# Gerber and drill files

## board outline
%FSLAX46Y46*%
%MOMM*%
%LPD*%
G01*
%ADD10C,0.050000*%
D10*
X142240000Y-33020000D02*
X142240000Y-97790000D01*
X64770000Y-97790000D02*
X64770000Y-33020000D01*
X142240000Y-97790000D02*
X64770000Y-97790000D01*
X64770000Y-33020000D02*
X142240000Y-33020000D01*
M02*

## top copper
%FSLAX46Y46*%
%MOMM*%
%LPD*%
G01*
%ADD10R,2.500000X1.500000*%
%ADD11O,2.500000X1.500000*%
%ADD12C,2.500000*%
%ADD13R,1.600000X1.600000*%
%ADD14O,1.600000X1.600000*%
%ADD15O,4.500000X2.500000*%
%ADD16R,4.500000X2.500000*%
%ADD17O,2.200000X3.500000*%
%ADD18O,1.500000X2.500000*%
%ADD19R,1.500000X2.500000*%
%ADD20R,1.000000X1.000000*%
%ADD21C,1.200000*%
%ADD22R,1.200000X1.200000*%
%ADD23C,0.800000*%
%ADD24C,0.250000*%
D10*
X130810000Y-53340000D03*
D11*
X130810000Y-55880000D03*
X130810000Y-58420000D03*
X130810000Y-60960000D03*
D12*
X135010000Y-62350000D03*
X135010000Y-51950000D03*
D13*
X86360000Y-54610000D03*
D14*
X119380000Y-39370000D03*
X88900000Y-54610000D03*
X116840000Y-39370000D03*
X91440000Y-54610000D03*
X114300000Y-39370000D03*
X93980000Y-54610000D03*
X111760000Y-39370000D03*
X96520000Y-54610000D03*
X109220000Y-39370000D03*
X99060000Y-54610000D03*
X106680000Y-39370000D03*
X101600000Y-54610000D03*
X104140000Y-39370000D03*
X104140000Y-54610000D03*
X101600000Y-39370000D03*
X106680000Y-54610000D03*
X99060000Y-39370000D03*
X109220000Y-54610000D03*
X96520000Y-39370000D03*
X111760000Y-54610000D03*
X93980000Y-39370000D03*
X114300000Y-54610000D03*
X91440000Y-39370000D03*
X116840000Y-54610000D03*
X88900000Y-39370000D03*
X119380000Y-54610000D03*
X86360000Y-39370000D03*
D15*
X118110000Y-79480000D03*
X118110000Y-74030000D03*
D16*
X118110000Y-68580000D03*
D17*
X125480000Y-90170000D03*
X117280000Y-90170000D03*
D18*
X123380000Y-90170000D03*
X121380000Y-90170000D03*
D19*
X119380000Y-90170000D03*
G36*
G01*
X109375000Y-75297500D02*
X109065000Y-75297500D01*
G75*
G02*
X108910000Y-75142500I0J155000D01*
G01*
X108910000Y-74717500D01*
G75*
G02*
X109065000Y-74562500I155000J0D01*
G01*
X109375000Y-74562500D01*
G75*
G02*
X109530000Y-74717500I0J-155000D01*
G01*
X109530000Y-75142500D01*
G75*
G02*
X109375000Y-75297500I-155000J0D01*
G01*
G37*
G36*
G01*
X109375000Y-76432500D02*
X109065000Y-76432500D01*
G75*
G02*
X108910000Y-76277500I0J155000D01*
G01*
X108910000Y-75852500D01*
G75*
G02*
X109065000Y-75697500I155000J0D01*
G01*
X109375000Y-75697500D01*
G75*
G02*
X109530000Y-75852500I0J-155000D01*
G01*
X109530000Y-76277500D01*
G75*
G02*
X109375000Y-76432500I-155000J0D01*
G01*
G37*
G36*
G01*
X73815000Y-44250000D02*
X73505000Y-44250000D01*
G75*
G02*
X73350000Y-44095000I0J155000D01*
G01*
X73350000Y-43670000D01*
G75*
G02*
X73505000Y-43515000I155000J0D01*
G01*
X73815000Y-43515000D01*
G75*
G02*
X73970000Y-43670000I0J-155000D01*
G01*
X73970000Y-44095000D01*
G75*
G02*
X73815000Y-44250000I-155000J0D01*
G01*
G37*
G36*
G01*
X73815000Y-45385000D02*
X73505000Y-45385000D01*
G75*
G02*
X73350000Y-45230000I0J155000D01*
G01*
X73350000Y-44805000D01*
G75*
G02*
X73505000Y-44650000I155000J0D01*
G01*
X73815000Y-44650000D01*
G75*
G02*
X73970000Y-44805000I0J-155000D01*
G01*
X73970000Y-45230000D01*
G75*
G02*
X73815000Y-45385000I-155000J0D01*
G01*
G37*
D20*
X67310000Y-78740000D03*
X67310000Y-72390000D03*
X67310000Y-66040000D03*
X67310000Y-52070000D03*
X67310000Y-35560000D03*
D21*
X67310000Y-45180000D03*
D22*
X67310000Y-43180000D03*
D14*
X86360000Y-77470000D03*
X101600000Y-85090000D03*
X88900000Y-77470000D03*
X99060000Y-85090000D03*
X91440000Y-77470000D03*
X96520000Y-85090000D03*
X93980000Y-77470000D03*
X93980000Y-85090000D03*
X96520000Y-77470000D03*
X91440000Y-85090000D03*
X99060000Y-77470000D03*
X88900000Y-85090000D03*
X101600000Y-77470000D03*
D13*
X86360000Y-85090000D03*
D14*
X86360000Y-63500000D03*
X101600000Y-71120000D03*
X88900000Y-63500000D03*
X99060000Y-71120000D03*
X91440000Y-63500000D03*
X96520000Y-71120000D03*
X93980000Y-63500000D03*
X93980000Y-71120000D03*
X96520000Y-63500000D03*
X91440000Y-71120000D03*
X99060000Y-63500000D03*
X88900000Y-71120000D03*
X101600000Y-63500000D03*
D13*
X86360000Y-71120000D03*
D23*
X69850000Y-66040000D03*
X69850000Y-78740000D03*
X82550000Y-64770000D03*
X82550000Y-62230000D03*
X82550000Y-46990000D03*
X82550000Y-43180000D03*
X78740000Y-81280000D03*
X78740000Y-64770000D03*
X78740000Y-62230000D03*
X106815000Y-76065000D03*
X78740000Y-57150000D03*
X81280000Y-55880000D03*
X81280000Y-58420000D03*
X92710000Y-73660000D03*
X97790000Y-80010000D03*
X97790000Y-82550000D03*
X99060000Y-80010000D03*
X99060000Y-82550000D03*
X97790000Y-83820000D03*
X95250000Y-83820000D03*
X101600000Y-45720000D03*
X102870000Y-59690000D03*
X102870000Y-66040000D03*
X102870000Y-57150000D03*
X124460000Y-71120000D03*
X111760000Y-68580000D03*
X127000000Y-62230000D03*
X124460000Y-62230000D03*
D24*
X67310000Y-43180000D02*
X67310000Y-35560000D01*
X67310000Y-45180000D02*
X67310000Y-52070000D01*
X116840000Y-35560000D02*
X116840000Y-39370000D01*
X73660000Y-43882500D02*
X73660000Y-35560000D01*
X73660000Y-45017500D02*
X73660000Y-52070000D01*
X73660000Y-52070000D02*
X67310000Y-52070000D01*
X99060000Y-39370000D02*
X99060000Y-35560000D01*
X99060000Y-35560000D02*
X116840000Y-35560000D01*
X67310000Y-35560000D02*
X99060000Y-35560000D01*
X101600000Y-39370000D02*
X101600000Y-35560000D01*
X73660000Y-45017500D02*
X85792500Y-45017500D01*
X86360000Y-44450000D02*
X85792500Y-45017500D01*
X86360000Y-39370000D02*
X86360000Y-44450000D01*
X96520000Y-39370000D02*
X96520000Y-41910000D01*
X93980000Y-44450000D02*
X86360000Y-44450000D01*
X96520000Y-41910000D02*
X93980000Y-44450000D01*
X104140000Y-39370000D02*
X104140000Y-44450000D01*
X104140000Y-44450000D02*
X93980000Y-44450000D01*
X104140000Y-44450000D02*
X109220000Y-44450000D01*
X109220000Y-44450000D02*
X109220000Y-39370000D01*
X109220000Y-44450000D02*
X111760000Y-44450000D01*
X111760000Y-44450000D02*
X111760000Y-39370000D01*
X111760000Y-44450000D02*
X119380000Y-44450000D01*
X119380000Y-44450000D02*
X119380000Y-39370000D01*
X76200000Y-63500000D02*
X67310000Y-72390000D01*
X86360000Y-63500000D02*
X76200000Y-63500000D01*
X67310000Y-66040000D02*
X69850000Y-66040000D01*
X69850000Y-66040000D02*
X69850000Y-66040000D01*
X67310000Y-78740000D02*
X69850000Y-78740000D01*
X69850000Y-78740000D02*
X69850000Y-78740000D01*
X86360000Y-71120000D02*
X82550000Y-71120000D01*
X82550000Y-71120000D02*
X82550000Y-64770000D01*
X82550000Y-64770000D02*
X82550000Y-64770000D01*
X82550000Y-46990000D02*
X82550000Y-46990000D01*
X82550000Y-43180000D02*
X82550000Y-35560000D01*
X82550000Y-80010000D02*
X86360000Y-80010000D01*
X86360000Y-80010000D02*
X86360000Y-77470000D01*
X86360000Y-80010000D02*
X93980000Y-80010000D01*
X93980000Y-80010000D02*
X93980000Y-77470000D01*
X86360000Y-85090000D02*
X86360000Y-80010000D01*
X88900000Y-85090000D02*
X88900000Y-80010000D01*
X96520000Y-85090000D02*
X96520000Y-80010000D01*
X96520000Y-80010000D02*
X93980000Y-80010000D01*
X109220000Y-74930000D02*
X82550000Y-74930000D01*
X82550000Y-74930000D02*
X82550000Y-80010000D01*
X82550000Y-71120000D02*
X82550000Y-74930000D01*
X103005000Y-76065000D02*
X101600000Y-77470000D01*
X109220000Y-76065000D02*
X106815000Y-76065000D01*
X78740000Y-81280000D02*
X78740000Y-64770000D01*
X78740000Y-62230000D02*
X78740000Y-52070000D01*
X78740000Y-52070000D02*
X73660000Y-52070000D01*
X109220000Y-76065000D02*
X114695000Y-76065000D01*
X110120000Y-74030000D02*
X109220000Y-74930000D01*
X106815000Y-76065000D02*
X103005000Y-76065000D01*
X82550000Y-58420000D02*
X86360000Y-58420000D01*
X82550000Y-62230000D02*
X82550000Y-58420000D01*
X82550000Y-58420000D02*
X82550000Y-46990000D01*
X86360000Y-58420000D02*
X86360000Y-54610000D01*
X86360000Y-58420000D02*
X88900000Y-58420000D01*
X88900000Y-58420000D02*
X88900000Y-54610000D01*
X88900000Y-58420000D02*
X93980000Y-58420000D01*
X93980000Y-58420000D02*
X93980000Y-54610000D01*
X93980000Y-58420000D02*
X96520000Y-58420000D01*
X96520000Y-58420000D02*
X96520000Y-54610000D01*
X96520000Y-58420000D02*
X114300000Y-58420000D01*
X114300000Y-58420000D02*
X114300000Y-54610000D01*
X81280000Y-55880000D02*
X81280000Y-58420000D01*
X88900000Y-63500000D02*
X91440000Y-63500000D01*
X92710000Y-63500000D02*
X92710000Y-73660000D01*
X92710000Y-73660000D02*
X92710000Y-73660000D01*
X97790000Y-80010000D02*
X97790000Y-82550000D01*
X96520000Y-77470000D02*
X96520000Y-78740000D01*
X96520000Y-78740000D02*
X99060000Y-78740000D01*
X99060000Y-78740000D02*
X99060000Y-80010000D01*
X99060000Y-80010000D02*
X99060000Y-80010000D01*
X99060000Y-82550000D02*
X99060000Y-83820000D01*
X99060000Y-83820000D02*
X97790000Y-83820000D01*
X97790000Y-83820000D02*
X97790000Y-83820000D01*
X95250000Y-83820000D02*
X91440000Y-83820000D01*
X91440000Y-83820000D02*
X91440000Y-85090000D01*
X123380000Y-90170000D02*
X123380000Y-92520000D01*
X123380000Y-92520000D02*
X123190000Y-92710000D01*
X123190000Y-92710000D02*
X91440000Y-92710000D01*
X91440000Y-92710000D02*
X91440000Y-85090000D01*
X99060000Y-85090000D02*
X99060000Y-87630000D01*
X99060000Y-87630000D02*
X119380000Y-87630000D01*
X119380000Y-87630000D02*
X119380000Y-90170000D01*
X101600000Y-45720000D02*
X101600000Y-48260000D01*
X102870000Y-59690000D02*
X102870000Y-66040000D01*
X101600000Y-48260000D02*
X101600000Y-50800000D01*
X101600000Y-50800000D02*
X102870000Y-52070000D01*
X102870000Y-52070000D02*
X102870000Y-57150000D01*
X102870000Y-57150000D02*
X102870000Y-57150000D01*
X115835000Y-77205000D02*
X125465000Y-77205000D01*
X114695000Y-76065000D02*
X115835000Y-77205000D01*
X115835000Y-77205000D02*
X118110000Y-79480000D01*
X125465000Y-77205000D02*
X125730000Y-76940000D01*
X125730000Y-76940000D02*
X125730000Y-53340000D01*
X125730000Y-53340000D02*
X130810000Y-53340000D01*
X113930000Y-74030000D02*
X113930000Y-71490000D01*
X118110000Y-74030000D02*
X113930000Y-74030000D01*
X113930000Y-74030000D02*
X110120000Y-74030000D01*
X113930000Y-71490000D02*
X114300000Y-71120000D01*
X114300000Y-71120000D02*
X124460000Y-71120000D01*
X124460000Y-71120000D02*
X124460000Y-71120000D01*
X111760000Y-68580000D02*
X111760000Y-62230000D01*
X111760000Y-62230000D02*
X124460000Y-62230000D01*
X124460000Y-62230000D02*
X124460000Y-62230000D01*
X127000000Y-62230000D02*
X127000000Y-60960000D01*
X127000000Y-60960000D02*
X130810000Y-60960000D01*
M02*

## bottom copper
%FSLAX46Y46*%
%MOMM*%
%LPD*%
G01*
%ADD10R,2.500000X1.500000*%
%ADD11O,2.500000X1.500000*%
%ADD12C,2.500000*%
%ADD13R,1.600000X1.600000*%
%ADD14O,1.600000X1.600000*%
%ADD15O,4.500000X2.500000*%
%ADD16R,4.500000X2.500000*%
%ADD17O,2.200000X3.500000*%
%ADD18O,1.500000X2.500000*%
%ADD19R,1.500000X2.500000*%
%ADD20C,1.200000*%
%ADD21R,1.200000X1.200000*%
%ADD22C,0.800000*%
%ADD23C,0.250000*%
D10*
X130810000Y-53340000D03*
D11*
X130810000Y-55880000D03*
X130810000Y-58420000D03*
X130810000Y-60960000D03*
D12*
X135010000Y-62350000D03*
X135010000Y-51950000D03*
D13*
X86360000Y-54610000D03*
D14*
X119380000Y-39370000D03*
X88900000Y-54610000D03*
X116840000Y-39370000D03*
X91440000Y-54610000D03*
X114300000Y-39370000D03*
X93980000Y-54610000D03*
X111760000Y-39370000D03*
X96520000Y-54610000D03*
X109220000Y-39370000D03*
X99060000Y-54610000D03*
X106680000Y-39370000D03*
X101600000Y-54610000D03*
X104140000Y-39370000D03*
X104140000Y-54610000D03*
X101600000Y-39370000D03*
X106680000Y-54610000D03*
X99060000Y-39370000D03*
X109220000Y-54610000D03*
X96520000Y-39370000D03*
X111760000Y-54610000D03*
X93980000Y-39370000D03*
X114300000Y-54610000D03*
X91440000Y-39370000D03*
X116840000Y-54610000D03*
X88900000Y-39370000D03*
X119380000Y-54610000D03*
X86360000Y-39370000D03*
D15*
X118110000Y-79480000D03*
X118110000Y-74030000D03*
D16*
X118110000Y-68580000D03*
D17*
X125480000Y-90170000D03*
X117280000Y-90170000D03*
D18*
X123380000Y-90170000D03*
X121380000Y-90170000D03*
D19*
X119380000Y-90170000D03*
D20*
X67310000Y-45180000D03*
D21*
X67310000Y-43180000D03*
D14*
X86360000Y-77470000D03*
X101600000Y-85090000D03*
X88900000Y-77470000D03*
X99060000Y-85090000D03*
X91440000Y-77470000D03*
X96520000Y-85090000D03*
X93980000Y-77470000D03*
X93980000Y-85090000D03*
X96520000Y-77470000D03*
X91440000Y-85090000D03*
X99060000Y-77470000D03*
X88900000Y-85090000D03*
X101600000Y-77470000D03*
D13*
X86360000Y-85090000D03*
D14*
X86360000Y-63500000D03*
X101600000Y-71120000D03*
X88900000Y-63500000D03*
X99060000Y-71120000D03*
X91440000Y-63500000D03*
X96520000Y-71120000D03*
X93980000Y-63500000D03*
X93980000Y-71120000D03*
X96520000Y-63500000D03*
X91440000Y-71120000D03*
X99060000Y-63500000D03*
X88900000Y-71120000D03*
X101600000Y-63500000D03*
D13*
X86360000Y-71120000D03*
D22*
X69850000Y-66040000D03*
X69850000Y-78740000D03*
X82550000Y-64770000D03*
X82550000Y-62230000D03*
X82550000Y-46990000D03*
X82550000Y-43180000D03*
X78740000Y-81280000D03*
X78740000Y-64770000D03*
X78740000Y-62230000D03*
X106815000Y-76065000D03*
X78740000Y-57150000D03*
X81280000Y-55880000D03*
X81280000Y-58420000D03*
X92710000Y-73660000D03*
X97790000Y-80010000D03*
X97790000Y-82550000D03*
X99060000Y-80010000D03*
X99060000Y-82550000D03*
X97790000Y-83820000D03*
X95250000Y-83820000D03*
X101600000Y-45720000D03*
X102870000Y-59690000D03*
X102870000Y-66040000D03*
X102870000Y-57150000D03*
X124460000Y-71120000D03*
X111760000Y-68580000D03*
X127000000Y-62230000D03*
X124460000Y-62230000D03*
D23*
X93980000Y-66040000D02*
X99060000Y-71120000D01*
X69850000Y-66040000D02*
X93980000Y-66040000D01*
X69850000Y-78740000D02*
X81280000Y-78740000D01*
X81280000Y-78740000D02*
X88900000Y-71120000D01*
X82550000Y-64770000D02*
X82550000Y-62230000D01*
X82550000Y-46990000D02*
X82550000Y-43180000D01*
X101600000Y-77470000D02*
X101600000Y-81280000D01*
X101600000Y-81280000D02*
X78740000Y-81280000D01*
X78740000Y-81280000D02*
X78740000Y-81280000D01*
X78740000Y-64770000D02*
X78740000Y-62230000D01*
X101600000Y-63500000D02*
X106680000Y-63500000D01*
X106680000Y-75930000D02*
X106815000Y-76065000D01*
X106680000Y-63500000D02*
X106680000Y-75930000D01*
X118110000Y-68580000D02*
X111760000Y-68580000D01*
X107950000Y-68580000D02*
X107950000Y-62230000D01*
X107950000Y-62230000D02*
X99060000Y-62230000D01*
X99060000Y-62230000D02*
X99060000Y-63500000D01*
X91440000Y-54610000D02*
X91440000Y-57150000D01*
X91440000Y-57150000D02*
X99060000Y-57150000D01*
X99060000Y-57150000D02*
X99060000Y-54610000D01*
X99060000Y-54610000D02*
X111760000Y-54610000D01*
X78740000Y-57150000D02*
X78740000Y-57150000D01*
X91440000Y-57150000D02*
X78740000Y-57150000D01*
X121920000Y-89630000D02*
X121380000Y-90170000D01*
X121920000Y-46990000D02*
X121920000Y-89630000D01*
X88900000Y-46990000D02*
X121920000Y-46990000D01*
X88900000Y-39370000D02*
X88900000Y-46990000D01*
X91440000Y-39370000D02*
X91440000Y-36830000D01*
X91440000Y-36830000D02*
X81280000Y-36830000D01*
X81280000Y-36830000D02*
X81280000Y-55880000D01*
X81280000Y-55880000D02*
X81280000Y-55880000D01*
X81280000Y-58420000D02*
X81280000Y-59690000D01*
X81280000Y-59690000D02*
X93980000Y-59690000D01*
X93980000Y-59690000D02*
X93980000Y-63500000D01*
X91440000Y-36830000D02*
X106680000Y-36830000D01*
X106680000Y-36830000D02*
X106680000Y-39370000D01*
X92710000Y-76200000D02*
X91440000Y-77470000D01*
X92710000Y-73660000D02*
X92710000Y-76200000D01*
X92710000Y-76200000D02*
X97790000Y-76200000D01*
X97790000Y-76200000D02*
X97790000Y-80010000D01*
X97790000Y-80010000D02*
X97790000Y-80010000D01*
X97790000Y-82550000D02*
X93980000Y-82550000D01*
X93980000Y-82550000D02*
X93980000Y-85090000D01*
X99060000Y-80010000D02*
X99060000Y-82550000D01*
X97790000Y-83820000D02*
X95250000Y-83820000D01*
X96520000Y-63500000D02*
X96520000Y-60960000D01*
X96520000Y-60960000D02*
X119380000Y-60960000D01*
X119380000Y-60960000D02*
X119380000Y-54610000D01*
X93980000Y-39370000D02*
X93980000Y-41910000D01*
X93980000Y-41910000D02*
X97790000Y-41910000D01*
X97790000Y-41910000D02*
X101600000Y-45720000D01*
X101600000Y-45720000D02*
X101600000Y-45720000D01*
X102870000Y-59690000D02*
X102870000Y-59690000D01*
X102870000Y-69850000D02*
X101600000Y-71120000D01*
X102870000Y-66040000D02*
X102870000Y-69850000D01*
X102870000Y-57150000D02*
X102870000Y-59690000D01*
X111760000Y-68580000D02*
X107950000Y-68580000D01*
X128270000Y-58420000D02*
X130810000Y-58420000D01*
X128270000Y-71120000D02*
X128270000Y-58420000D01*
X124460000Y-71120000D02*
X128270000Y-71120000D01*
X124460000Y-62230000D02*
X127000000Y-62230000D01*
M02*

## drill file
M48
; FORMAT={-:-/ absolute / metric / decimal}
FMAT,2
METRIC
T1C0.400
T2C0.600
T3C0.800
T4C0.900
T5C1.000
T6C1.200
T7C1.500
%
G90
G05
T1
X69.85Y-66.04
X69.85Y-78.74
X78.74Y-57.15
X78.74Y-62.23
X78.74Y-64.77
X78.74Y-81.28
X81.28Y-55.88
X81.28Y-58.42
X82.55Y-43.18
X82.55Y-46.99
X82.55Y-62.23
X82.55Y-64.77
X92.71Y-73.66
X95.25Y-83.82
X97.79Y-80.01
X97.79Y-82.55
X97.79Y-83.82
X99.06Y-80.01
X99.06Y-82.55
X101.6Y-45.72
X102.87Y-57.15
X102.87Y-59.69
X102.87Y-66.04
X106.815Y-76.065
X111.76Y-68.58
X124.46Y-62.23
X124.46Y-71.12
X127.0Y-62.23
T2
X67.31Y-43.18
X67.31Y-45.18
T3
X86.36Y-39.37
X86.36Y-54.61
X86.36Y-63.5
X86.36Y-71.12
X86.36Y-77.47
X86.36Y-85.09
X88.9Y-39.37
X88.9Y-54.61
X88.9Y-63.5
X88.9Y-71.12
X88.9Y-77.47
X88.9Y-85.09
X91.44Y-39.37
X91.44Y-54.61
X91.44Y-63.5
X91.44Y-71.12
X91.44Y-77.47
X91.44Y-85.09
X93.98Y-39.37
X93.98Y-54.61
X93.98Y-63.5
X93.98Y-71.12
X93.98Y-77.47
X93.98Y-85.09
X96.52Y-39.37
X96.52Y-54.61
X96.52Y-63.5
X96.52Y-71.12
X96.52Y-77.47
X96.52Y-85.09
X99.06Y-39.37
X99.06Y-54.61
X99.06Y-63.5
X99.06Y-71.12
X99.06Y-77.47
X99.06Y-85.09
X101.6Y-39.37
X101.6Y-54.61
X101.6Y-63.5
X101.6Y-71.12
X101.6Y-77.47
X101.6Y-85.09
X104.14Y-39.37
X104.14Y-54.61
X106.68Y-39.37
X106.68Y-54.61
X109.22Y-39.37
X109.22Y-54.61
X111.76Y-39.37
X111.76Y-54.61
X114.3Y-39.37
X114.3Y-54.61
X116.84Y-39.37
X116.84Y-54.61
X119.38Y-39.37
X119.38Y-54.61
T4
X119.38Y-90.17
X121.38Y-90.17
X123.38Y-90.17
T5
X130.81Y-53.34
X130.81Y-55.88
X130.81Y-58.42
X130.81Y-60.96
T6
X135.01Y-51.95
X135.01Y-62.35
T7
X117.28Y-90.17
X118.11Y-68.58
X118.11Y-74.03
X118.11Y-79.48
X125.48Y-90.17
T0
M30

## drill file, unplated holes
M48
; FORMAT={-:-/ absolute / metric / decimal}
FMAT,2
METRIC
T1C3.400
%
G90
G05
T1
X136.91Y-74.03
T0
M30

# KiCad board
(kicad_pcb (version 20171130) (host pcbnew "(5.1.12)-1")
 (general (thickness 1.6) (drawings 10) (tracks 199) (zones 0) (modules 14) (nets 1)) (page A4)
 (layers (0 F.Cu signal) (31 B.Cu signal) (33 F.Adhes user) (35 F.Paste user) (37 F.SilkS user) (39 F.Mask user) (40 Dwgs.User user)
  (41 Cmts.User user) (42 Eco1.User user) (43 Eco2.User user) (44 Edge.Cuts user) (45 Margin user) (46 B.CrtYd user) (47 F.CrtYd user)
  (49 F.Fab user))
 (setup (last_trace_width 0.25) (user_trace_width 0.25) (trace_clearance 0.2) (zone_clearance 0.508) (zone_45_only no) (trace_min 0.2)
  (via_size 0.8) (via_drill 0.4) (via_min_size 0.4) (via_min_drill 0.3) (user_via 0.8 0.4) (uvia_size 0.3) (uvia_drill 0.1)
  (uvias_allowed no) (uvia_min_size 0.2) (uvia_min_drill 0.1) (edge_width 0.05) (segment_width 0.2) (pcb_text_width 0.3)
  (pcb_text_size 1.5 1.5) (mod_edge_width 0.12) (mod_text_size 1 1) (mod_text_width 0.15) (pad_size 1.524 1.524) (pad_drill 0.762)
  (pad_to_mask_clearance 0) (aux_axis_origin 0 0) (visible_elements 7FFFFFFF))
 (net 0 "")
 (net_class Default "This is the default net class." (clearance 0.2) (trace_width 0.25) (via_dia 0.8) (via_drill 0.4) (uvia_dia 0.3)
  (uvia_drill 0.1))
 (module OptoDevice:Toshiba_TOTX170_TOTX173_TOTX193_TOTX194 (layer F.Cu) (at 130.81 53.34 270)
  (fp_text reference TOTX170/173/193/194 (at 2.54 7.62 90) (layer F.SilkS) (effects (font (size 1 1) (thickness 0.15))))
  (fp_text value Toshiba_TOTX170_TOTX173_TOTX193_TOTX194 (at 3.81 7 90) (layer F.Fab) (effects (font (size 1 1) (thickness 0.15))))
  (pad 1 thru_hole rect (at 0 0 270) (size 1.5 2.5) (drill 1) (layers *.Cu *.Mask))
  (pad 2 thru_hole oval (at 2.54 0 270) (size 1.5 2.5) (drill 1) (layers *.Cu *.Mask))
  (pad 3 thru_hole oval (at 5.08 0 270) (size 1.5 2.5) (drill 1) (layers *.Cu *.Mask))
  (pad 4 thru_hole oval (at 7.62 0 270) (size 1.5 2.5) (drill 1) (layers *.Cu *.Mask))
  (pad 5 thru_hole circle (at 9.01 -4.2 270) (size 2.5 2.5) (drill 1.2) (layers *.Cu *.Mask))
  (pad 6 thru_hole circle (at -1.39 -4.2 270) (size 2.5 2.5) (drill 1.2) (layers *.Cu *.Mask)))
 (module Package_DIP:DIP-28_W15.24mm (layer F.Cu) (at 86.36 54.61 90)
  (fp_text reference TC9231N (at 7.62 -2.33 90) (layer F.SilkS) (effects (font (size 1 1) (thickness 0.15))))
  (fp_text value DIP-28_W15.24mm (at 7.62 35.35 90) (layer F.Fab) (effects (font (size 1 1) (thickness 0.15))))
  (pad 1 thru_hole rect (at 0 0 90) (size 1.6 1.6) (drill 0.8) (layers *.Cu *.Mask))
  (pad 15 thru_hole oval (at 15.24 33.02 90) (size 1.6 1.6) (drill 0.8) (layers *.Cu *.Mask))
  (pad 2 thru_hole oval (at 0 2.54 90) (size 1.6 1.6) (drill 0.8) (layers *.Cu *.Mask))
  (pad 16 thru_hole oval (at 15.24 30.48 90) (size 1.6 1.6) (drill 0.8) (layers *.Cu *.Mask))
  (pad 3 thru_hole oval (at 0 5.08 90) (size 1.6 1.6) (drill 0.8) (layers *.Cu *.Mask))
  (pad 17 thru_hole oval (at 15.24 27.94 90) (size 1.6 1.6) (drill 0.8) (layers *.Cu *.Mask))
  (pad 4 thru_hole oval (at 0 7.62 90) (size 1.6 1.6) (drill 0.8) (layers *.Cu *.Mask))
  (pad 18 thru_hole oval (at 15.24 25.4 90) (size 1.6 1.6) (drill 0.8) (layers *.Cu *.Mask))
  (pad 5 thru_hole oval (at 0 10.16 90) (size 1.6 1.6) (drill 0.8) (layers *.Cu *.Mask))
  (pad 19 thru_hole oval (at 15.24 22.86 90) (size 1.6 1.6) (drill 0.8) (layers *.Cu *.Mask))
  (pad 6 thru_hole oval (at 0 12.7 90) (size 1.6 1.6) (drill 0.8) (layers *.Cu *.Mask))
  (pad 20 thru_hole oval (at 15.24 20.32 90) (size 1.6 1.6) (drill 0.8) (layers *.Cu *.Mask))
  (pad 7 thru_hole oval (at 0 15.24 90) (size 1.6 1.6) (drill 0.8) (layers *.Cu *.Mask))
  (pad 21 thru_hole oval (at 15.24 17.78 90) (size 1.6 1.6) (drill 0.8) (layers *.Cu *.Mask))
  (pad 8 thru_hole oval (at 0 17.78 90) (size 1.6 1.6) (drill 0.8) (layers *.Cu *.Mask))
  (pad 22 thru_hole oval (at 15.24 15.24 90) (size 1.6 1.6) (drill 0.8) (layers *.Cu *.Mask))
  (pad 9 thru_hole oval (at 0 20.32 90) (size 1.6 1.6) (drill 0.8) (layers *.Cu *.Mask))
  (pad 23 thru_hole oval (at 15.24 12.7 90) (size 1.6 1.6) (drill 0.8) (layers *.Cu *.Mask))
  (pad 10 thru_hole oval (at 0 22.86 90) (size 1.6 1.6) (drill 0.8) (layers *.Cu *.Mask))
  (pad 24 thru_hole oval (at 15.24 10.16 90) (size 1.6 1.6) (drill 0.8) (layers *.Cu *.Mask))
  (pad 11 thru_hole oval (at 0 25.4 90) (size 1.6 1.6) (drill 0.8) (layers *.Cu *.Mask))
  (pad 25 thru_hole oval (at 15.24 7.62 90) (size 1.6 1.6) (drill 0.8) (layers *.Cu *.Mask))
  (pad 12 thru_hole oval (at 0 27.94 90) (size 1.6 1.6) (drill 0.8) (layers *.Cu *.Mask))
  (pad 26 thru_hole oval (at 15.24 5.08 90) (size 1.6 1.6) (drill 0.8) (layers *.Cu *.Mask))
  (pad 13 thru_hole oval (at 0 30.48 90) (size 1.6 1.6) (drill 0.8) (layers *.Cu *.Mask))
  (pad 27 thru_hole oval (at 15.24 2.54 90) (size 1.6 1.6) (drill 0.8) (layers *.Cu *.Mask))
  (pad 14 thru_hole oval (at 0 33.02 90) (size 1.6 1.6) (drill 0.8) (layers *.Cu *.Mask))
  (pad 28 thru_hole oval (at 15.24 0 90) (size 1.6 1.6) (drill 0.8) (layers *.Cu *.Mask)))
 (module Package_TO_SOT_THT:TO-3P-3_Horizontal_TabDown (layer F.Cu) (at 118.11 68.58 270)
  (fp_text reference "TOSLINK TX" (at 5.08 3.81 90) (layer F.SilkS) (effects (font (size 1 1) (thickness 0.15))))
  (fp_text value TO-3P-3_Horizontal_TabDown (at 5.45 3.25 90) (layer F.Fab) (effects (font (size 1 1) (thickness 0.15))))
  (pad 3 thru_hole oval (at 10.9 0 270) (size 2.5 4.5) (drill 1.5) (layers *.Cu *.Mask))
  (pad 2 thru_hole oval (at 5.45 0 270) (size 2.5 4.5) (drill 1.5) (layers *.Cu *.Mask))
  (pad 1 thru_hole rect (at 0 0 270) (size 2.5 4.5) (drill 1.5) (layers *.Cu *.Mask))
  (pad "" np_thru_hole oval (at 5.45 -18.8 270) (size 3.4 3.4) (drill 3.4) (layers *.Cu *.Mask)))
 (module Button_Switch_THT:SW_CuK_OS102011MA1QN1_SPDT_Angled (layer F.Cu) (at 119.38 90.17)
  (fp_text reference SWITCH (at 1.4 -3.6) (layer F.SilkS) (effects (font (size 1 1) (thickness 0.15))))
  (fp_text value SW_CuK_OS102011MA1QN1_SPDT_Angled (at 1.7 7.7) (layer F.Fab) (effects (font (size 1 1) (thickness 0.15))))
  (pad "" thru_hole oval (at 6.1 0) (size 2.2 3.5) (drill 1.5) (layers *.Cu *.Mask))
  (pad "" thru_hole oval (at -2.1 0) (size 2.2 3.5) (drill 1.5) (layers *.Cu *.Mask))
  (pad 3 thru_hole oval (at 4 0) (size 1.5 2.5) (drill 0.9) (layers *.Cu *.Mask))
  (pad 2 thru_hole oval (at 2 0) (size 1.5 2.5) (drill 0.9) (layers *.Cu *.Mask))
  (pad 1 thru_hole rect (at 0 0) (size 1.5 2.5) (drill 0.9) (layers *.Cu *.Mask)))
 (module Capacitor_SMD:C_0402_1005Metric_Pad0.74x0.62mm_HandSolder (layer F.Cu) (at 109.22 75.4975 90)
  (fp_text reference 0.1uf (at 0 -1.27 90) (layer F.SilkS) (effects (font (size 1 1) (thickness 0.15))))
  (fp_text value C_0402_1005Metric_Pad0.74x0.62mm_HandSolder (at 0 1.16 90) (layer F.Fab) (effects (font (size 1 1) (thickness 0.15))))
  (pad 2 smd roundrect (at 0.5675 0 90) (size 0.735 0.62) (layers F.Cu F.Paste F.Mask) (roundrect_rratio 0.25))
  (pad 1 smd roundrect (at -0.5675 0 90) (size 0.735 0.62) (layers F.Cu F.Paste F.Mask) (roundrect_rratio 0.25)))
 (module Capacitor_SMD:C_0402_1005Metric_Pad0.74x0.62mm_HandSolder (layer F.Cu) (at 73.66 44.45 90)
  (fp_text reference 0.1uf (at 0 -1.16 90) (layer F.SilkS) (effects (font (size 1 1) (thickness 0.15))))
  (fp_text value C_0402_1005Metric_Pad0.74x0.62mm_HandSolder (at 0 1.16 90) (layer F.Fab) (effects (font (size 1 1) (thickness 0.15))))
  (pad 2 smd roundrect (at 0.5675 0 90) (size 0.735 0.62) (layers F.Cu F.Paste F.Mask) (roundrect_rratio 0.25))
  (pad 1 smd roundrect (at -0.5675 0 90) (size 0.735 0.62) (layers F.Cu F.Paste F.Mask) (roundrect_rratio 0.25)))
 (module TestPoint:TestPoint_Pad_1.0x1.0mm (layer F.Cu) (at 67.31 78.74)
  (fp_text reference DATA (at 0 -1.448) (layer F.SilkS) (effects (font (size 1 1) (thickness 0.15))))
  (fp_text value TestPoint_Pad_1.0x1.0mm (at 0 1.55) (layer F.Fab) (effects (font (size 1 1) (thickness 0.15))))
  (pad 1 smd rect (at 0 0) (size 1 1) (layers F.Cu F.Mask)))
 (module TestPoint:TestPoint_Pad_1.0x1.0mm (layer F.Cu) (at 67.31 72.39)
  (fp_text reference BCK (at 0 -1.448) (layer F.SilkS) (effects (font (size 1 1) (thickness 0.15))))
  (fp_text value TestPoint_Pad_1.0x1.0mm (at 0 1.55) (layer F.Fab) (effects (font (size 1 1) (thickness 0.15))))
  (pad 1 smd rect (at 0 0) (size 1 1) (layers F.Cu F.Mask)))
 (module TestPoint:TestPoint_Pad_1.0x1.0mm (layer F.Cu) (at 67.31 66.04)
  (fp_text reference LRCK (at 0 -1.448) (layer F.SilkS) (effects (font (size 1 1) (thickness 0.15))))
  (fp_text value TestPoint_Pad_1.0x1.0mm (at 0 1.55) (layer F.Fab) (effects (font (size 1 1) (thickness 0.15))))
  (pad 1 smd rect (at 0 0) (size 1 1) (layers F.Cu F.Mask)))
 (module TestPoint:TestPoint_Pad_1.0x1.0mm (layer F.Cu) (at 67.31 52.07)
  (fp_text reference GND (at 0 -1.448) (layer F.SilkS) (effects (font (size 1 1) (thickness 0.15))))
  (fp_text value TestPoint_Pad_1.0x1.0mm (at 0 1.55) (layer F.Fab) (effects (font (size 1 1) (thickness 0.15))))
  (pad 1 smd rect (at 0 0) (size 1 1) (layers F.Cu F.Mask)))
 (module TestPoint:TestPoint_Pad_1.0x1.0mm (layer F.Cu) (at 67.31 35.56)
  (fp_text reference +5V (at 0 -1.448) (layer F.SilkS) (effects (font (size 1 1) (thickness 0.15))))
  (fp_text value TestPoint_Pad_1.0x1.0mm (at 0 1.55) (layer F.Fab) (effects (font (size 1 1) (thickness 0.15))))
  (pad 1 smd rect (at 0 0) (size 1 1) (layers F.Cu F.Mask)))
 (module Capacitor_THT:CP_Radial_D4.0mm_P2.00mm (layer F.Cu) (at 67.31 43.18 270)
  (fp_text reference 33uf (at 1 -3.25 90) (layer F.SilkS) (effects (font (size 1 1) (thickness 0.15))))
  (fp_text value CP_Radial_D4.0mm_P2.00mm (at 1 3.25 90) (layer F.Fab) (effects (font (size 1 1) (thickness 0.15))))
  (pad 2 thru_hole circle (at 2 0 270) (size 1.2 1.2) (drill 0.6) (layers *.Cu *.Mask))
  (pad 1 thru_hole rect (at 0 0 270) (size 1.2 1.2) (drill 0.6) (layers *.Cu *.Mask)))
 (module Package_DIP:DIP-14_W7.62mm (layer F.Cu) (at 86.36 85.09 90)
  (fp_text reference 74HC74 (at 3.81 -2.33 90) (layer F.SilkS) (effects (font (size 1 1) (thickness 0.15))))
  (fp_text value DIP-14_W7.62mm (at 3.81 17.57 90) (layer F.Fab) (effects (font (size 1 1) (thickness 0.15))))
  (pad 14 thru_hole oval (at 7.62 0 90) (size 1.6 1.6) (drill 0.8) (layers *.Cu *.Mask))
  (pad 7 thru_hole oval (at 0 15.24 90) (size 1.6 1.6) (drill 0.8) (layers *.Cu *.Mask))
  (pad 13 thru_hole oval (at 7.62 2.54 90) (size 1.6 1.6) (drill 0.8) (layers *.Cu *.Mask))
  (pad 6 thru_hole oval (at 0 12.7 90) (size 1.6 1.6) (drill 0.8) (layers *.Cu *.Mask))
  (pad 12 thru_hole oval (at 7.62 5.08 90) (size 1.6 1.6) (drill 0.8) (layers *.Cu *.Mask))
  (pad 5 thru_hole oval (at 0 10.16 90) (size 1.6 1.6) (drill 0.8) (layers *.Cu *.Mask))
  (pad 11 thru_hole oval (at 7.62 7.62 90) (size 1.6 1.6) (drill 0.8) (layers *.Cu *.Mask))
  (pad 4 thru_hole oval (at 0 7.62 90) (size 1.6 1.6) (drill 0.8) (layers *.Cu *.Mask))
  (pad 10 thru_hole oval (at 7.62 10.16 90) (size 1.6 1.6) (drill 0.8) (layers *.Cu *.Mask))
  (pad 3 thru_hole oval (at 0 5.08 90) (size 1.6 1.6) (drill 0.8) (layers *.Cu *.Mask))
  (pad 9 thru_hole oval (at 7.62 12.7 90) (size 1.6 1.6) (drill 0.8) (layers *.Cu *.Mask))
  (pad 2 thru_hole oval (at 0 2.54 90) (size 1.6 1.6) (drill 0.8) (layers *.Cu *.Mask))
  (pad 8 thru_hole oval (at 7.62 15.24 90) (size 1.6 1.6) (drill 0.8) (layers *.Cu *.Mask))
  (pad 1 thru_hole rect (at 0 0 90) (size 1.6 1.6) (drill 0.8) (layers *.Cu *.Mask)))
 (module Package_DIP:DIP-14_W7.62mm (layer F.Cu) (at 86.36 71.12 90)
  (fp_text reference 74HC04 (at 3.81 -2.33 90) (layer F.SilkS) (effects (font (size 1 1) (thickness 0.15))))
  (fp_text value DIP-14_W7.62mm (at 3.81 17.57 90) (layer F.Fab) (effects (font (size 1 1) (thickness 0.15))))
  (pad 14 thru_hole oval (at 7.62 0 90) (size 1.6 1.6) (drill 0.8) (layers *.Cu *.Mask))
  (pad 7 thru_hole oval (at 0 15.24 90) (size 1.6 1.6) (drill 0.8) (layers *.Cu *.Mask))
  (pad 13 thru_hole oval (at 7.62 2.54 90) (size 1.6 1.6) (drill 0.8) (layers *.Cu *.Mask))
  (pad 6 thru_hole oval (at 0 12.7 90) (size 1.6 1.6) (drill 0.8) (layers *.Cu *.Mask))
  (pad 12 thru_hole oval (at 7.62 5.08 90) (size 1.6 1.6) (drill 0.8) (layers *.Cu *.Mask))
  (pad 5 thru_hole oval (at 0 10.16 90) (size 1.6 1.6) (drill 0.8) (layers *.Cu *.Mask))
  (pad 11 thru_hole oval (at 7.62 7.62 90) (size 1.6 1.6) (drill 0.8) (layers *.Cu *.Mask))
  (pad 4 thru_hole oval (at 0 7.62 90) (size 1.6 1.6) (drill 0.8) (layers *.Cu *.Mask))
  (pad 10 thru_hole oval (at 7.62 10.16 90) (size 1.6 1.6) (drill 0.8) (layers *.Cu *.Mask))
  (pad 3 thru_hole oval (at 0 5.08 90) (size 1.6 1.6) (drill 0.8) (layers *.Cu *.Mask))
  (pad 9 thru_hole oval (at 7.62 12.7 90) (size 1.6 1.6) (drill 0.8) (layers *.Cu *.Mask))
  (pad 2 thru_hole oval (at 0 2.54 90) (size 1.6 1.6) (drill 0.8) (layers *.Cu *.Mask))
  (pad 8 thru_hole oval (at 7.62 15.24 90) (size 1.6 1.6) (drill 0.8) (layers *.Cu *.Mask))
  (pad 1 thru_hole rect (at 0 0 90) (size 1.6 1.6) (drill 0.8) (layers *.Cu *.Mask)))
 (gr_line (start 142.24 33.02) (end 142.24 97.79) (layer Edge.Cuts) (width 0.05))
 (gr_line (start 64.77 97.79) (end 64.77 33.02) (layer Edge.Cuts) (width 0.05))
 (gr_line (start 142.24 97.79) (end 64.77 97.79) (layer Edge.Cuts) (width 0.05))
 (gr_line (start 64.77 33.02) (end 142.24 33.02) (layer Edge.Cuts) (width 0.05))
 (segment (start 67.31 43.18) (end 67.31 35.56) (width 0.25) (layer F.Cu) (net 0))
 (segment (start 67.31 45.18) (end 67.31 52.07) (width 0.25) (layer F.Cu) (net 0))
 (segment (start 116.84 35.56) (end 116.84 39.37) (width 0.25) (layer F.Cu) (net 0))
 (segment (start 73.66 43.8825) (end 73.66 35.56) (width 0.25) (layer F.Cu) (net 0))
 (segment (start 73.66 45.0175) (end 73.66 52.07) (width 0.25) (layer F.Cu) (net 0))
 (segment (start 73.66 52.07) (end 67.31 52.07) (width 0.25) (layer F.Cu) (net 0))
 (segment (start 99.06 39.37) (end 99.06 35.56) (width 0.25) (layer F.Cu) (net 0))
 (segment (start 99.06 35.56) (end 116.84 35.56) (width 0.25) (layer F.Cu) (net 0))
 (segment (start 67.31 35.56) (end 99.06 35.56) (width 0.25) (layer F.Cu) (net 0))
 (segment (start 101.6 39.37) (end 101.6 35.56) (width 0.25) (layer F.Cu) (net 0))
 (segment (start 73.66 45.0175) (end 85.7925 45.0175) (width 0.25) (layer F.Cu) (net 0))
 (segment (start 86.36 44.45) (end 85.7925 45.0175) (width 0.25) (layer F.Cu) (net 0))
 (segment (start 86.36 39.37) (end 86.36 44.45) (width 0.25) (layer F.Cu) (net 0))
 (segment (start 96.52 39.37) (end 96.52 41.91) (width 0.25) (layer F.Cu) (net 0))
 (segment (start 93.98 44.45) (end 86.36 44.45) (width 0.25) (layer F.Cu) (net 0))
 (segment (start 96.52 41.91) (end 93.98 44.45) (width 0.25) (layer F.Cu) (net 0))
 (segment (start 104.14 39.37) (end 104.14 44.45) (width 0.25) (layer F.Cu) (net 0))
 (segment (start 104.14 44.45) (end 93.98 44.45) (width 0.25) (layer F.Cu) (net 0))
 (segment (start 104.14 44.45) (end 109.22 44.45) (width 0.25) (layer F.Cu) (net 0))
 (segment (start 109.22 44.45) (end 109.22 39.37) (width 0.25) (layer F.Cu) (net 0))
 (segment (start 109.22 44.45) (end 111.76 44.45) (width 0.25) (layer F.Cu) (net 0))
 (segment (start 111.76 44.45) (end 111.76 39.37) (width 0.25) (layer F.Cu) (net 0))
 (segment (start 111.76 44.45) (end 119.38 44.45) (width 0.25) (layer F.Cu) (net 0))
 (segment (start 119.38 44.45) (end 119.38 39.37) (width 0.25) (layer F.Cu) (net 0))
 (segment (start 76.2 63.5) (end 67.31 72.39) (width 0.25) (layer F.Cu) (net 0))
 (segment (start 86.36 63.5) (end 76.2 63.5) (width 0.25) (layer F.Cu) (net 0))
 (segment (start 67.31 66.04) (end 69.85 66.04) (width 0.25) (layer F.Cu) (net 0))
 (segment (start 69.85 66.04) (end 69.85 66.04) (width 0.25) (layer F.Cu) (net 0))
 (via (at 69.85 66.04) (size 0.8) (drill 0.4) (layers F.Cu B.Cu) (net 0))
 (segment (start 93.98 66.04) (end 99.06 71.12) (width 0.25) (layer B.Cu) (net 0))
 (segment (start 69.85 66.04) (end 93.98 66.04) (width 0.25) (layer B.Cu) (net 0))
 (segment (start 67.31 78.74) (end 69.85 78.74) (width 0.25) (layer F.Cu) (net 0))
 (segment (start 69.85 78.74) (end 69.85 78.74) (width 0.25) (layer F.Cu) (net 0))
 (via (at 69.85 78.74) (size 0.8) (drill 0.4) (layers F.Cu B.Cu) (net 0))
 (segment (start 69.85 78.74) (end 81.28 78.74) (width 0.25) (layer B.Cu) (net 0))
 (segment (start 81.28 78.74) (end 88.9 71.12) (width 0.25) (layer B.Cu) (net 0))
 (segment (start 86.36 71.12) (end 82.55 71.12) (width 0.25) (layer F.Cu) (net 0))
 (segment (start 82.55 71.12) (end 82.55 64.77) (width 0.25) (layer F.Cu) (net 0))
 (segment (start 82.55 64.77) (end 82.55 64.77) (width 0.25) (layer F.Cu) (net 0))
 (via (at 82.55 64.77) (size 0.8) (drill 0.4) (layers F.Cu B.Cu) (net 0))
 (via (at 82.55 62.23) (size 0.8) (drill 0.4) (layers F.Cu B.Cu) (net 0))
 (segment (start 82.55 64.77) (end 82.55 62.23) (width 0.25) (layer B.Cu) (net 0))
 (segment (start 82.55 46.99) (end 82.55 46.99) (width 0.25) (layer F.Cu) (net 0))
 (via (at 82.55 46.99) (size 0.8) (drill 0.4) (layers F.Cu B.Cu) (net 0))
 (via (at 82.55 43.18) (size 0.8) (drill 0.4) (layers F.Cu B.Cu) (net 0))
 (segment (start 82.55 46.99) (end 82.55 43.18) (width 0.25) (layer B.Cu) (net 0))
 (segment (start 82.55 43.18) (end 82.55 35.56) (width 0.25) (layer F.Cu) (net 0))
 (segment (start 82.55 80.01) (end 86.36 80.01) (width 0.25) (layer F.Cu) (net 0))
 (segment (start 86.36 80.01) (end 86.36 77.47) (width 0.25) (layer F.Cu) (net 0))
 (segment (start 86.36 80.01) (end 93.98 80.01) (width 0.25) (layer F.Cu) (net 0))
 (segment (start 93.98 80.01) (end 93.98 77.47) (width 0.25) (layer F.Cu) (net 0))
 (segment (start 86.36 85.09) (end 86.36 80.01) (width 0.25) (layer F.Cu) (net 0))
 (segment (start 88.9 85.09) (end 88.9 80.01) (width 0.25) (layer F.Cu) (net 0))
 (segment (start 96.52 85.09) (end 96.52 80.01) (width 0.25) (layer F.Cu) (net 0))
 (segment (start 96.52 80.01) (end 93.98 80.01) (width 0.25) (layer F.Cu) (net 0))
 (segment (start 109.22 74.93) (end 82.55 74.93) (width 0.25) (layer F.Cu) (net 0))
 (segment (start 82.55 74.93) (end 82.55 80.01) (width 0.25) (layer F.Cu) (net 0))
 (segment (start 82.55 71.12) (end 82.55 74.93) (width 0.25) (layer F.Cu) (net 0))
 (segment (start 103.005 76.065) (end 101.6 77.47) (width 0.25) (layer F.Cu) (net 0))
 (segment (start 109.22 76.065) (end 106.815 76.065) (width 0.25) (layer F.Cu) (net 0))
 (segment (start 101.6 77.47) (end 101.6 81.28) (width 0.25) (layer B.Cu) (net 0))
 (segment (start 101.6 81.28) (end 78.74 81.28) (width 0.25) (layer B.Cu) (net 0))
 (segment (start 78.74 81.28) (end 78.74 81.28) (width 0.25) (layer B.Cu) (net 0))
 (via (at 78.74 81.28) (size 0.8) (drill 0.4) (layers F.Cu B.Cu) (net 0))
 (via (at 78.74 64.77) (size 0.8) (drill 0.4) (layers F.Cu B.Cu) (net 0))
 (via (at 78.74 62.23) (size 0.8) (drill 0.4) (layers F.Cu B.Cu) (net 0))
 (segment (start 78.74 81.28) (end 78.74 64.77) (width 0.25) (layer F.Cu) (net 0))
 (segment (start 78.74 64.77) (end 78.74 62.23) (width 0.25) (layer B.Cu) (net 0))
 (segment (start 78.74 62.23) (end 78.74 52.07) (width 0.25) (layer F.Cu) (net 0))
 (segment (start 78.74 52.07) (end 73.66 52.07) (width 0.25) (layer F.Cu) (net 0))
 (segment (start 109.22 76.065) (end 114.695 76.065) (width 0.25) (layer F.Cu) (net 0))
 (segment (start 110.12 74.03) (end 109.22 74.93) (width 0.25) (layer F.Cu) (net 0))
 (segment (start 106.815 76.065) (end 103.005 76.065) (width 0.25) (layer F.Cu) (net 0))
 (via (at 106.815 76.065) (size 0.8) (drill 0.4) (layers F.Cu B.Cu) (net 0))
 (segment (start 101.6 63.5) (end 106.68 63.5) (width 0.25) (layer B.Cu) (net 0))
 (segment (start 106.68 75.93) (end 106.815 76.065) (width 0.25) (layer B.Cu) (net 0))
 (segment (start 106.68 63.5) (end 106.68 75.93) (width 0.25) (layer B.Cu) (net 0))
 (segment (start 118.11 68.58) (end 111.76 68.58) (width 0.25) (layer B.Cu) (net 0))
 (segment (start 107.95 68.58) (end 107.95 62.23) (width 0.25) (layer B.Cu) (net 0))
 (segment (start 107.95 62.23) (end 99.06 62.23) (width 0.25) (layer B.Cu) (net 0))
 (segment (start 99.06 62.23) (end 99.06 63.5) (width 0.25) (layer B.Cu) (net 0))
 (segment (start 82.55 58.42) (end 86.36 58.42) (width 0.25) (layer F.Cu) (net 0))
 (segment (start 82.55 62.23) (end 82.55 58.42) (width 0.25) (layer F.Cu) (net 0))
 (segment (start 82.55 58.42) (end 82.55 46.99) (width 0.25) (layer F.Cu) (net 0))
 (segment (start 86.36 58.42) (end 86.36 54.61) (width 0.25) (layer F.Cu) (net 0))
 (segment (start 86.36 58.42) (end 88.9 58.42) (width 0.25) (layer F.Cu) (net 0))
 (segment (start 88.9 58.42) (end 88.9 54.61) (width 0.25) (layer F.Cu) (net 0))
 (segment (start 88.9 58.42) (end 93.98 58.42) (width 0.25) (layer F.Cu) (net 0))
 (segment (start 93.98 58.42) (end 93.98 54.61) (width 0.25) (layer F.Cu) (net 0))
 (segment (start 93.98 58.42) (end 96.52 58.42) (width 0.25) (layer F.Cu) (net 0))
 (segment (start 96.52 58.42) (end 96.52 54.61) (width 0.25) (layer F.Cu) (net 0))
 (segment (start 96.52 58.42) (end 114.3 58.42) (width 0.25) (layer F.Cu) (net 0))
 (segment (start 114.3 58.42) (end 114.3 54.61) (width 0.25) (layer F.Cu) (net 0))
 (segment (start 91.44 54.61) (end 91.44 57.15) (width 0.25) (layer B.Cu) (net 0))
 (segment (start 91.44 57.15) (end 99.06 57.15) (width 0.25) (layer B.Cu) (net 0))
 (segment (start 99.06 57.15) (end 99.06 54.61) (width 0.25) (layer B.Cu) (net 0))
 (segment (start 99.06 54.61) (end 111.76 54.61) (width 0.25) (layer B.Cu) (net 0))
 (segment (start 78.74 57.15) (end 78.74 57.15) (width 0.25) (layer B.Cu) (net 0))
 (via (at 78.74 57.15) (size 0.8) (drill 0.4) (layers F.Cu B.Cu) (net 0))
 (segment (start 91.44 57.15) (end 78.74 57.15) (width 0.25) (layer B.Cu) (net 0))
 (segment (start 121.92 89.63) (end 121.38 90.17) (width 0.25) (layer B.Cu) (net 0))
 (segment (start 121.92 46.99) (end 121.92 89.63) (width 0.25) (layer B.Cu) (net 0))
 (segment (start 88.9 46.99) (end 121.92 46.99) (width 0.25) (layer B.Cu) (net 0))
 (segment (start 88.9 39.37) (end 88.9 46.99) (width 0.25) (layer B.Cu) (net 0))
 (segment (start 91.44 39.37) (end 91.44 36.83) (width 0.25) (layer B.Cu) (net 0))
 (segment (start 91.44 36.83) (end 81.28 36.83) (width 0.25) (layer B.Cu) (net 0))
 (segment (start 81.28 36.83) (end 81.28 55.88) (width 0.25) (layer B.Cu) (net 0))
 (segment (start 81.28 55.88) (end 81.28 55.88) (width 0.25) (layer B.Cu) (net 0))
 (via (at 81.28 55.88) (size 0.8) (drill 0.4) (layers F.Cu B.Cu) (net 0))
 (via (at 81.28 58.42) (size 0.8) (drill 0.4) (layers F.Cu B.Cu) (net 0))
 (segment (start 81.28 55.88) (end 81.28 58.42) (width 0.25) (layer F.Cu) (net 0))
 (segment (start 81.28 58.42) (end 81.28 59.69) (width 0.25) (layer B.Cu) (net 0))
 (segment (start 81.28 59.69) (end 93.98 59.69) (width 0.25) (layer B.Cu) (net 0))
 (segment (start 93.98 59.69) (end 93.98 63.5) (width 0.25) (layer B.Cu) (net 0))
 (segment (start 91.44 36.83) (end 106.68 36.83) (width 0.25) (layer B.Cu) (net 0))
 (segment (start 106.68 36.83) (end 106.68 39.37) (width 0.25) (layer B.Cu) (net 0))
 (segment (start 88.9 63.5) (end 91.44 63.5) (width 0.25) (layer F.Cu) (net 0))
 (segment (start 92.71 63.5) (end 92.71 73.66) (width 0.25) (layer F.Cu) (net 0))
 (segment (start 92.71 73.66) (end 92.71 73.66) (width 0.25) (layer F.Cu) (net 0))
 (via (at 92.71 73.66) (size 0.8) (drill 0.4) (layers F.Cu B.Cu) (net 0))
 (segment (start 92.71 76.2) (end 91.44 77.47) (width 0.25) (layer B.Cu) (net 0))
 (segment (start 92.71 73.66) (end 92.71 76.2) (width 0.25) (layer B.Cu) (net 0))
 (segment (start 92.71 76.2) (end 97.79 76.2) (width 0.25) (layer B.Cu) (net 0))
 (segment (start 97.79 76.2) (end 97.79 80.01) (width 0.25) (layer B.Cu) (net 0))
 (segment (start 97.79 80.01) (end 97.79 80.01) (width 0.25) (layer B.Cu) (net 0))
 (via (at 97.79 80.01) (size 0.8) (drill 0.4) (layers F.Cu B.Cu) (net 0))
 (via (at 97.79 82.55) (size 0.8) (drill 0.4) (layers F.Cu B.Cu) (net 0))
 (segment (start 97.79 80.01) (end 97.79 82.55) (width 0.25) (layer F.Cu) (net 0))
 (segment (start 97.79 82.55) (end 93.98 82.55) (width 0.25) (layer B.Cu) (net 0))
 (segment (start 93.98 82.55) (end 93.98 85.09) (width 0.25) (layer B.Cu) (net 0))
 (segment (start 96.52 77.47) (end 96.52 78.74) (width 0.25) (layer F.Cu) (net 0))
 (segment (start 96.52 78.74) (end 99.06 78.74) (width 0.25) (layer F.Cu) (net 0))
 (segment (start 99.06 78.74) (end 99.06 80.01) (width 0.25) (layer F.Cu) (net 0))
 (segment (start 99.06 80.01) (end 99.06 80.01) (width 0.25) (layer F.Cu) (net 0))
 (via (at 99.06 80.01) (size 0.8) (drill 0.4) (layers F.Cu B.Cu) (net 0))
 (via (at 99.06 82.55) (size 0.8) (drill 0.4) (layers F.Cu B.Cu) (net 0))
 (segment (start 99.06 80.01) (end 99.06 82.55) (width 0.25) (layer B.Cu) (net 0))
 (segment (start 99.06 82.55) (end 99.06 83.82) (width 0.25) (layer F.Cu) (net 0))
 (segment (start 99.06 83.82) (end 97.79 83.82) (width 0.25) (layer F.Cu) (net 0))
 (segment (start 97.79 83.82) (end 97.79 83.82) (width 0.25) (layer F.Cu) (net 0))
 (via (at 97.79 83.82) (size 0.8) (drill 0.4) (layers F.Cu B.Cu) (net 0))
 (via (at 95.25 83.82) (size 0.8) (drill 0.4) (layers F.Cu B.Cu) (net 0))
 (segment (start 97.79 83.82) (end 95.25 83.82) (width 0.25) (layer B.Cu) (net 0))
 (segment (start 95.25 83.82) (end 91.44 83.82) (width 0.25) (layer F.Cu) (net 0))
 (segment (start 91.44 83.82) (end 91.44 85.09) (width 0.25) (layer F.Cu) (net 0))
 (segment (start 123.38 90.17) (end 123.38 92.52) (width 0.25) (layer F.Cu) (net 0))
 (segment (start 123.38 92.52) (end 123.19 92.71) (width 0.25) (layer F.Cu) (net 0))
 (segment (start 123.19 92.71) (end 91.44 92.71) (width 0.25) (layer F.Cu) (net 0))
 (segment (start 91.44 92.71) (end 91.44 85.09) (width 0.25) (layer F.Cu) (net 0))
 (segment (start 99.06 85.09) (end 99.06 87.63) (width 0.25) (layer F.Cu) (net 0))
 (segment (start 99.06 87.63) (end 119.38 87.63) (width 0.25) (layer F.Cu) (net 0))
 (segment (start 119.38 87.63) (end 119.38 90.17) (width 0.25) (layer F.Cu) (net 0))
 (segment (start 96.52 63.5) (end 96.52 60.96) (width 0.25) (layer B.Cu) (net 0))
 (segment (start 96.52 60.96) (end 119.38 60.96) (width 0.25) (layer B.Cu) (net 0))
 (segment (start 119.38 60.96) (end 119.38 54.61) (width 0.25) (layer B.Cu) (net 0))
 (segment (start 93.98 39.37) (end 93.98 41.91) (width 0.25) (layer B.Cu) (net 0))
 (segment (start 93.98 41.91) (end 97.79 41.91) (width 0.25) (layer B.Cu) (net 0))
 (segment (start 97.79 41.91) (end 101.6 45.72) (width 0.25) (layer B.Cu) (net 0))
 (segment (start 101.6 45.72) (end 101.6 45.72) (width 0.25) (layer B.Cu) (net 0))
 (via (at 101.6 45.72) (size 0.8) (drill 0.4) (layers F.Cu B.Cu) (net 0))
 (segment (start 101.6 45.72) (end 101.6 48.26) (width 0.25) (layer F.Cu) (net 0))
 (segment (start 102.87 59.69) (end 102.87 59.69) (width 0.25) (layer B.Cu) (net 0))
 (via (at 102.87 59.69) (size 0.8) (drill 0.4) (layers F.Cu B.Cu) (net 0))
 (via (at 102.87 66.04) (size 0.8) (drill 0.4) (layers F.Cu B.Cu) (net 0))
 (segment (start 102.87 59.69) (end 102.87 66.04) (width 0.25) (layer F.Cu) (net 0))
 (segment (start 102.87 69.85) (end 101.6 71.12) (width 0.25) (layer B.Cu) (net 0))
 (segment (start 102.87 66.04) (end 102.87 69.85) (width 0.25) (layer B.Cu) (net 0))
 (segment (start 101.6 48.26) (end 101.6 50.8) (width 0.25) (layer F.Cu) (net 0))
 (segment (start 101.6 50.8) (end 102.87 52.07) (width 0.25) (layer F.Cu) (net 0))
 (segment (start 102.87 52.07) (end 102.87 57.15) (width 0.25) (layer F.Cu) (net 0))
 (segment (start 102.87 57.15) (end 102.87 57.15) (width 0.25) (layer F.Cu) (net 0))
 (via (at 102.87 57.15) (size 0.8) (drill 0.4) (layers F.Cu B.Cu) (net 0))
 (segment (start 102.87 57.15) (end 102.87 59.69) (width 0.25) (layer B.Cu) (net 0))
 (segment (start 115.835 77.205) (end 125.465 77.205) (width 0.25) (layer F.Cu) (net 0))
 (segment (start 114.695 76.065) (end 115.835 77.205) (width 0.25) (layer F.Cu) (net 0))
 (segment (start 115.835 77.205) (end 118.11 79.48) (width 0.25) (layer F.Cu) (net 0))
 (segment (start 125.465 77.205) (end 125.73 76.94) (width 0.25) (layer F.Cu) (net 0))
 (segment (start 125.73 76.94) (end 125.73 53.34) (width 0.25) (layer F.Cu) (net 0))
 (segment (start 125.73 53.34) (end 130.81 53.34) (width 0.25) (layer F.Cu) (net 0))
 (segment (start 113.93 74.03) (end 113.93 71.49) (width 0.25) (layer F.Cu) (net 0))
 (segment (start 118.11 74.03) (end 113.93 74.03) (width 0.25) (layer F.Cu) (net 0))
 (segment (start 113.93 74.03) (end 110.12 74.03) (width 0.25) (layer F.Cu) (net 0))
 (segment (start 113.93 71.49) (end 114.3 71.12) (width 0.25) (layer F.Cu) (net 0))
 (segment (start 114.3 71.12) (end 124.46 71.12) (width 0.25) (layer F.Cu) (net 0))
 (segment (start 124.46 71.12) (end 124.46 71.12) (width 0.25) (layer F.Cu) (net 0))
 (via (at 124.46 71.12) (size 0.8) (drill 0.4) (layers F.Cu B.Cu) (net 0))
 (segment (start 111.76 68.58) (end 107.95 68.58) (width 0.25) (layer B.Cu) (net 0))
 (via (at 111.76 68.58) (size 0.8) (drill 0.4) (layers F.Cu B.Cu) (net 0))
 (segment (start 111.76 68.58) (end 111.76 62.23) (width 0.25) (layer F.Cu) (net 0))
 (segment (start 111.76 62.23) (end 124.46 62.23) (width 0.25) (layer F.Cu) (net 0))
 (segment (start 128.27 58.42) (end 130.81 58.42) (width 0.25) (layer B.Cu) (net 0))
 (segment (start 128.27 71.12) (end 128.27 58.42) (width 0.25) (layer B.Cu) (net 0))
 (segment (start 124.46 71.12) (end 128.27 71.12) (width 0.25) (layer B.Cu) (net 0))
 (via (at 127 62.23) (size 0.8) (drill 0.4) (layers F.Cu B.Cu) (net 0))
 (segment (start 124.46 62.23) (end 124.46 62.23) (width 0.25) (layer F.Cu) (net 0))
 (via (at 124.46 62.23) (size 0.8) (drill 0.4) (layers F.Cu B.Cu) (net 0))
 (segment (start 124.46 62.23) (end 127 62.23) (width 0.25) (layer B.Cu) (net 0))
 (segment (start 127 62.23) (end 127 60.96) (width 0.25) (layer F.Cu) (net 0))
 (segment (start 127 60.96) (end 130.81 60.96) (width 0.25) (layer F.Cu) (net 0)))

